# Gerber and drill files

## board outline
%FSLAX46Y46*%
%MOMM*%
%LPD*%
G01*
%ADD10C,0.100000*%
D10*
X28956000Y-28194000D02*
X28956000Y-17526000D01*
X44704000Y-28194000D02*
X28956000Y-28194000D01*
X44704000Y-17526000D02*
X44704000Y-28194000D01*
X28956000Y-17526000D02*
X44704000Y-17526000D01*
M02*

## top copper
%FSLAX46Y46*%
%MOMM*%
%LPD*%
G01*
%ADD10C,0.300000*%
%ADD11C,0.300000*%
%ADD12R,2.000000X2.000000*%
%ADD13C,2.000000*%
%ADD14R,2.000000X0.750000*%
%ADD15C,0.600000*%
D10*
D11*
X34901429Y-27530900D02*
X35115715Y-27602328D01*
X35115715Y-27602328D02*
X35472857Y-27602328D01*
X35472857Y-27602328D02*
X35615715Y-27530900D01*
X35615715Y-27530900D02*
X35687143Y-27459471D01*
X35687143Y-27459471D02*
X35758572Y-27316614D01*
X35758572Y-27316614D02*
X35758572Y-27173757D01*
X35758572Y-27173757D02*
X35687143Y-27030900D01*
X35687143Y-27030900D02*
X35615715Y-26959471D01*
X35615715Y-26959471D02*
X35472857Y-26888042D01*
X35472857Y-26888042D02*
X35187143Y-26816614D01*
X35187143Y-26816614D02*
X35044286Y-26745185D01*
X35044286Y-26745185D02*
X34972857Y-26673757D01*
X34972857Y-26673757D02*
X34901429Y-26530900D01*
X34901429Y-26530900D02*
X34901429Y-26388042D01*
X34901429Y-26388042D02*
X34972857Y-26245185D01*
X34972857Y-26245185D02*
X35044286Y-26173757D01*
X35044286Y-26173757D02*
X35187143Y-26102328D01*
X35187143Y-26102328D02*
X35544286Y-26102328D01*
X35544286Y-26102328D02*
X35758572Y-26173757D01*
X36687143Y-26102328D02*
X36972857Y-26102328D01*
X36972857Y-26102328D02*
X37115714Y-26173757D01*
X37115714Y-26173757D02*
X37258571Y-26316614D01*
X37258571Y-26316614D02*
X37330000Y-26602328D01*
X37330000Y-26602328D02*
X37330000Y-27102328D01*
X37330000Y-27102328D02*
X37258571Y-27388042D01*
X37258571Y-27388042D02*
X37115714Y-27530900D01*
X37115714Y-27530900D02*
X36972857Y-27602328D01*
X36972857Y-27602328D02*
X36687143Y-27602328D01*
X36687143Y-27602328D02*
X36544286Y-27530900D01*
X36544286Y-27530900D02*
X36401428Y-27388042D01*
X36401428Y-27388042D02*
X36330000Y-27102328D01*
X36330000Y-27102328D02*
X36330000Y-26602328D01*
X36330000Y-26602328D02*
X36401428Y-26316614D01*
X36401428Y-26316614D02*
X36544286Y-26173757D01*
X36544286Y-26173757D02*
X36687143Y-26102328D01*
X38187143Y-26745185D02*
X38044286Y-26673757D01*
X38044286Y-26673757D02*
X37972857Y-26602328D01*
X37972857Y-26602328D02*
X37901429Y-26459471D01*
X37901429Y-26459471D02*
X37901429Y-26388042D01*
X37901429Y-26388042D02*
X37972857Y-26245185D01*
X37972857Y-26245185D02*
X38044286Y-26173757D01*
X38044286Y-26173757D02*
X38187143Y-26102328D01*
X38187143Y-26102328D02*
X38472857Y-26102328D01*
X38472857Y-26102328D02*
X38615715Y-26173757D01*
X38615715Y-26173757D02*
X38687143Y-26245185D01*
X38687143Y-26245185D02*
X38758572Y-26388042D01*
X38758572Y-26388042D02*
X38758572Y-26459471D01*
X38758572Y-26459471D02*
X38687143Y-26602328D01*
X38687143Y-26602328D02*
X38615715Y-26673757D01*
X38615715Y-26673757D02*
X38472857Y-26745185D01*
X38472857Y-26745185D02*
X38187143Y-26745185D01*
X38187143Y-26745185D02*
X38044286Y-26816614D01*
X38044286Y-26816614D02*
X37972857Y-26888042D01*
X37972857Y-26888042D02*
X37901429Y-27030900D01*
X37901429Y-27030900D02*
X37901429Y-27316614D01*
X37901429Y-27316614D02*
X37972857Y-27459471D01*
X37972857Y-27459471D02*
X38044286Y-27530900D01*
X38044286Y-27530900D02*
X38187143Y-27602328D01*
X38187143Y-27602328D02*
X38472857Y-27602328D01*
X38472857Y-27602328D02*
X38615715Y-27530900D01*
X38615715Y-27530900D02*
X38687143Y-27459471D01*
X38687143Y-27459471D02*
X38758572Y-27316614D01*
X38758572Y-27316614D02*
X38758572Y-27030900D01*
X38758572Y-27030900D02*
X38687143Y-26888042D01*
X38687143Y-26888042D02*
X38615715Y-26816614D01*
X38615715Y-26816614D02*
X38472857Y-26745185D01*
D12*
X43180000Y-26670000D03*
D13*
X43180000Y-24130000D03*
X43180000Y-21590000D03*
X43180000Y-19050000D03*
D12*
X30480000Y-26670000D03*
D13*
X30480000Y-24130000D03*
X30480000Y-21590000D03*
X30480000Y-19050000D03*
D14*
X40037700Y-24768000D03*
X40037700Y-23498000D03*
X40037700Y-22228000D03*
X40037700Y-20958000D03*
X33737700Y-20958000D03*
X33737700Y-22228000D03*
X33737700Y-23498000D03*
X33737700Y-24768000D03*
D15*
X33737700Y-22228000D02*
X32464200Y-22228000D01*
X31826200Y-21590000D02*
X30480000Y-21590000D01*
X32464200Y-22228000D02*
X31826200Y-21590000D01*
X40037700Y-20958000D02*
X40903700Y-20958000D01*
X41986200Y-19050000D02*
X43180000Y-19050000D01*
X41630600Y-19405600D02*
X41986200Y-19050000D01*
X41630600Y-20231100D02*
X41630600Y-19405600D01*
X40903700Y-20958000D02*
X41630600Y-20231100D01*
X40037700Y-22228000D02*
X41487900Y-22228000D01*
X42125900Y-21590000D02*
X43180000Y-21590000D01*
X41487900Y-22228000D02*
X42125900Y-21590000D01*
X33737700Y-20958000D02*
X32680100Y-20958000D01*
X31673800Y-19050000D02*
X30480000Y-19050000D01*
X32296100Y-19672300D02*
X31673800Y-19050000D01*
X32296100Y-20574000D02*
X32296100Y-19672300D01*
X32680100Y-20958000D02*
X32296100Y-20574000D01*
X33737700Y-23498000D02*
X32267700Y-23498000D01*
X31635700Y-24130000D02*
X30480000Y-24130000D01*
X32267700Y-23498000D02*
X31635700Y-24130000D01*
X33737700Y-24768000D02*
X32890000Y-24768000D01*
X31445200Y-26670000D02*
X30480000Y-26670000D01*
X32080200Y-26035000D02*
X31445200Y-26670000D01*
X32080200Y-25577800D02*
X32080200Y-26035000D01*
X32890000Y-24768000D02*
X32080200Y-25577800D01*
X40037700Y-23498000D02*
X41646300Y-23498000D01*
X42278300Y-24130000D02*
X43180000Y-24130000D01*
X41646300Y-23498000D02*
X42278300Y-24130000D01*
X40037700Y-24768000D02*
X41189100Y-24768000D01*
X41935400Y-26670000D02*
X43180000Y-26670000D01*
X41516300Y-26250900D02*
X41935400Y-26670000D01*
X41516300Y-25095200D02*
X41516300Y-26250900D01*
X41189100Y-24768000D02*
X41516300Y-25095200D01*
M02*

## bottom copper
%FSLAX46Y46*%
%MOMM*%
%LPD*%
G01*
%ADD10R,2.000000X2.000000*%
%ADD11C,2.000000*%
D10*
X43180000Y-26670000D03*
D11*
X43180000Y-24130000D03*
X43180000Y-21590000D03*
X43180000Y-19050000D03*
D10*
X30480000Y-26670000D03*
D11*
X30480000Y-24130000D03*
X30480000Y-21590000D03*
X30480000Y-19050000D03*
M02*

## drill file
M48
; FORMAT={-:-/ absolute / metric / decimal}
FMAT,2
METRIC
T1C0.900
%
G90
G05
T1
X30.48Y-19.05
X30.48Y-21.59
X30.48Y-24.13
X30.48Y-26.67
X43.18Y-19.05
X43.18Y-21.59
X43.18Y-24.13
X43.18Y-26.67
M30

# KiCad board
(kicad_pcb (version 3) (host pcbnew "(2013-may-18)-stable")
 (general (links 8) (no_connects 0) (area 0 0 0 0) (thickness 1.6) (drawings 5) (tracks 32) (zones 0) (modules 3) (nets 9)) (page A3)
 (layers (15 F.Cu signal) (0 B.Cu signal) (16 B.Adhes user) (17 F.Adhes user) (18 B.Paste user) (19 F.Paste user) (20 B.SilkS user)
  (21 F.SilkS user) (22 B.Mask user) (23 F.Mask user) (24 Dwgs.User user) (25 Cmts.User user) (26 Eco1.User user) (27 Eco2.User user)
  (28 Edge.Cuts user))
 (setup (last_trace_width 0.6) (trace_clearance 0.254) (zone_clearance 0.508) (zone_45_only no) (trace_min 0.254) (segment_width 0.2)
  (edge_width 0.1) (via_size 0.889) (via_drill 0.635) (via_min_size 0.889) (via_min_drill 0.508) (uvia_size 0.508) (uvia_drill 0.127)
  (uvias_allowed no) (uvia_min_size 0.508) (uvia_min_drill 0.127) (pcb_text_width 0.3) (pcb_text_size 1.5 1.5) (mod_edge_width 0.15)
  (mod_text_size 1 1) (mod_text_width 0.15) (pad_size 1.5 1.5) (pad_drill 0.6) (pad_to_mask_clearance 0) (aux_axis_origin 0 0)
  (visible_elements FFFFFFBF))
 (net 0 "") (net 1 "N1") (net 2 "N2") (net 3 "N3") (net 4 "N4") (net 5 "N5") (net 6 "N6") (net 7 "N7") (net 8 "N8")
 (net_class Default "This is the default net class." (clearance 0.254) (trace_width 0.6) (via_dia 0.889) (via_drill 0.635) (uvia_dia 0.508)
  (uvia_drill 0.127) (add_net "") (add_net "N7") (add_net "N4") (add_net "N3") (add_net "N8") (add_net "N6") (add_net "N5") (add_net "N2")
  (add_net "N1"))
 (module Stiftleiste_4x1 (layer F.Cu) (at 43.18 22.86 90)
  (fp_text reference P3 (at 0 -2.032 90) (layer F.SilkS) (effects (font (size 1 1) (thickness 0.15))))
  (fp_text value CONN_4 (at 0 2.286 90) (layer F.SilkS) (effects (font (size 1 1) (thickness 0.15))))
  (pad 1 thru_hole rect (at -3.81 0 90) (size 2 2) (drill 0.9) (layers *.Cu *.Mask F.SilkS) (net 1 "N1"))
  (pad 2 thru_hole circle (at -1.27 0 90) (size 2 2) (drill 0.9) (layers *.Cu *.Mask F.SilkS) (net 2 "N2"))
  (pad 3 thru_hole circle (at 1.27 0 90) (size 2 2) (drill 0.9) (layers *.Cu *.Mask F.SilkS) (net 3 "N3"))
  (pad 4 thru_hole circle (at 3.81 0 90) (size 2 2) (drill 0.9) (layers *.Cu *.Mask F.SilkS) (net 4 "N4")))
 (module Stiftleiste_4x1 (layer F.Cu) (at 30.48 22.86 90)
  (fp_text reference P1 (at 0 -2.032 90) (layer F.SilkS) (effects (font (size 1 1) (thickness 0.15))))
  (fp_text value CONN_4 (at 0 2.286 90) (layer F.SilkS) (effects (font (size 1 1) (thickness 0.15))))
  (pad 1 thru_hole rect (at -3.81 0 90) (size 2 2) (drill 0.9) (layers *.Cu *.Mask F.SilkS) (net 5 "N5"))
  (pad 2 thru_hole circle (at -1.27 0 90) (size 2 2) (drill 0.9) (layers *.Cu *.Mask F.SilkS) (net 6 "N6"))
  (pad 3 thru_hole circle (at 1.27 0 90) (size 2 2) (drill 0.9) (layers *.Cu *.Mask F.SilkS) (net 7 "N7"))
  (pad 4 thru_hole circle (at 3.81 0 90) (size 2 2) (drill 0.9) (layers *.Cu *.Mask F.SilkS) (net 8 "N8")))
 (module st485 (layer F.Cu) (at 34.9377 22.86 90)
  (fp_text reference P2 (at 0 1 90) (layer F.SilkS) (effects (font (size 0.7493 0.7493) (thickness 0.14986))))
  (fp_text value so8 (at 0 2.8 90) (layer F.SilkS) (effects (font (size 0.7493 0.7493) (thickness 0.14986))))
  (pad 1 smd rect (at -1.908 5.1 90) (size 0.75 2) (layers F.Cu F.Paste F.Mask) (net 1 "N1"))
  (pad 2 smd rect (at -0.638 5.1 90) (size 0.75 2) (layers F.Cu F.Paste F.Mask) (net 2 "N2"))
  (pad 3 smd rect (at 0.632 5.1 90) (size 0.75 2) (layers F.Cu F.Paste F.Mask) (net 3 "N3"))
  (pad 4 smd rect (at 1.902 5.1 90) (size 0.75 2) (layers F.Cu F.Paste F.Mask) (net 4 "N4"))
  (pad 5 smd rect (at 1.902 -1.2 90) (size 0.75 2) (layers F.Cu F.Paste F.Mask) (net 8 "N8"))
  (pad 6 smd rect (at 0.632 -1.2 90) (size 0.75 2) (layers F.Cu F.Paste F.Mask) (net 7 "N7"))
  (pad 7 smd rect (at -0.638 -1.2 90) (size 0.75 2) (layers F.Cu F.Paste F.Mask) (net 6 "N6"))
  (pad 8 smd rect (at -1.908 -1.2 90) (size 0.75 2) (layers F.Cu F.Paste F.Mask) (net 5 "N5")))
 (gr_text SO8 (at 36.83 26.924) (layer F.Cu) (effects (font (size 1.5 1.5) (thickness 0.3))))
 (gr_line (start 28.956 28.194) (end 28.956 17.526) (angle 90) (layer Edge.Cuts) (width 0.1))
 (gr_line (start 44.704 28.194) (end 28.956 28.194) (angle 90) (layer Edge.Cuts) (width 0.1))
 (gr_line (start 44.704 17.526) (end 44.704 28.194) (angle 90) (layer Edge.Cuts) (width 0.1))
 (gr_line (start 28.956 17.526) (end 44.704 17.526) (angle 90) (layer Edge.Cuts) (width 0.1))
 (segment (start 33.7377 22.228) (end 32.4642 22.228) (width 0.6) (layer F.Cu) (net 7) (status 400000))
 (segment (start 31.8262 21.59) (end 30.48 21.59) (width 0.6) (layer F.Cu) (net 7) (status 800000))
 (segment (start 32.4642 22.228) (end 31.8262 21.59) (width 0.6) (layer F.Cu) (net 7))
 (segment (start 40.0377 20.958) (end 40.9037 20.958) (width 0.6) (layer F.Cu) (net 4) (status C00000))
 (segment (start 41.9862 19.05) (end 43.18 19.05) (width 0.6) (layer F.Cu) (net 4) (status 800000))
 (segment (start 41.6306 19.4056) (end 41.9862 19.05) (width 0.6) (layer F.Cu) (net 4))
 (segment (start 41.6306 20.2311) (end 41.6306 19.4056) (width 0.6) (layer F.Cu) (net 4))
 (segment (start 40.9037 20.958) (end 41.6306 20.2311) (width 0.6) (layer F.Cu) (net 4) (status 400000))
 (segment (start 40.0377 22.228) (end 41.4879 22.228) (width 0.6) (layer F.Cu) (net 3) (status 400000))
 (segment (start 42.1259 21.59) (end 43.18 21.59) (width 0.6) (layer F.Cu) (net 3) (status 800000))
 (segment (start 41.4879 22.228) (end 42.1259 21.59) (width 0.6) (layer F.Cu) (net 3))
 (segment (start 33.7377 20.958) (end 32.6801 20.958) (width 0.6) (layer F.Cu) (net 8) (status 400000))
 (segment (start 31.6738 19.05) (end 30.48 19.05) (width 0.6) (layer F.Cu) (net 8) (status 800000))
 (segment (start 32.2961 19.6723) (end 31.6738 19.05) (width 0.6) (layer F.Cu) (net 8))
 (segment (start 32.2961 20.574) (end 32.2961 19.6723) (width 0.6) (layer F.Cu) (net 8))
 (segment (start 32.6801 20.958) (end 32.2961 20.574) (width 0.6) (layer F.Cu) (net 8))
 (segment (start 33.7377 23.498) (end 32.2677 23.498) (width 0.6) (layer F.Cu) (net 6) (status 400000))
 (segment (start 31.6357 24.13) (end 30.48 24.13) (width 0.6) (layer F.Cu) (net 6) (status 800000))
 (segment (start 32.2677 23.498) (end 31.6357 24.13) (width 0.6) (layer F.Cu) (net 6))
 (segment (start 33.7377 24.768) (end 32.89 24.768) (width 0.6) (layer F.Cu) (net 5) (status C00000))
 (segment (start 31.4452 26.67) (end 30.48 26.67) (width 0.6) (layer F.Cu) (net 5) (status C00000))
 (segment (start 32.0802 26.035) (end 31.4452 26.67) (width 0.6) (layer F.Cu) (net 5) (status 800000))
 (segment (start 32.0802 25.5778) (end 32.0802 26.035) (width 0.6) (layer F.Cu) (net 5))
 (segment (start 32.89 24.768) (end 32.0802 25.5778) (width 0.6) (layer F.Cu) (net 5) (status 400000))
 (segment (start 40.0377 23.498) (end 41.6463 23.498) (width 0.6) (layer F.Cu) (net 2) (status 400000))
 (segment (start 42.2783 24.13) (end 43.18 24.13) (width 0.6) (layer F.Cu) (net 2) (status C00000))
 (segment (start 41.6463 23.498) (end 42.2783 24.13) (width 0.6) (layer F.Cu) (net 2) (status 800000))
 (segment (start 40.0377 24.768) (end 41.1891 24.768) (width 0.6) (layer F.Cu) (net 1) (status 400000))
 (segment (start 41.9354 26.67) (end 43.18 26.67) (width 0.6) (layer F.Cu) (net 1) (status 800000))
 (segment (start 41.5163 26.2509) (end 41.9354 26.67) (width 0.6) (layer F.Cu) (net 1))
 (segment (start 41.5163 25.0952) (end 41.5163 26.2509) (width 0.6) (layer F.Cu) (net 1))
 (segment (start 41.1891 24.768) (end 41.5163 25.0952) (width 0.6) (layer F.Cu) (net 1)))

